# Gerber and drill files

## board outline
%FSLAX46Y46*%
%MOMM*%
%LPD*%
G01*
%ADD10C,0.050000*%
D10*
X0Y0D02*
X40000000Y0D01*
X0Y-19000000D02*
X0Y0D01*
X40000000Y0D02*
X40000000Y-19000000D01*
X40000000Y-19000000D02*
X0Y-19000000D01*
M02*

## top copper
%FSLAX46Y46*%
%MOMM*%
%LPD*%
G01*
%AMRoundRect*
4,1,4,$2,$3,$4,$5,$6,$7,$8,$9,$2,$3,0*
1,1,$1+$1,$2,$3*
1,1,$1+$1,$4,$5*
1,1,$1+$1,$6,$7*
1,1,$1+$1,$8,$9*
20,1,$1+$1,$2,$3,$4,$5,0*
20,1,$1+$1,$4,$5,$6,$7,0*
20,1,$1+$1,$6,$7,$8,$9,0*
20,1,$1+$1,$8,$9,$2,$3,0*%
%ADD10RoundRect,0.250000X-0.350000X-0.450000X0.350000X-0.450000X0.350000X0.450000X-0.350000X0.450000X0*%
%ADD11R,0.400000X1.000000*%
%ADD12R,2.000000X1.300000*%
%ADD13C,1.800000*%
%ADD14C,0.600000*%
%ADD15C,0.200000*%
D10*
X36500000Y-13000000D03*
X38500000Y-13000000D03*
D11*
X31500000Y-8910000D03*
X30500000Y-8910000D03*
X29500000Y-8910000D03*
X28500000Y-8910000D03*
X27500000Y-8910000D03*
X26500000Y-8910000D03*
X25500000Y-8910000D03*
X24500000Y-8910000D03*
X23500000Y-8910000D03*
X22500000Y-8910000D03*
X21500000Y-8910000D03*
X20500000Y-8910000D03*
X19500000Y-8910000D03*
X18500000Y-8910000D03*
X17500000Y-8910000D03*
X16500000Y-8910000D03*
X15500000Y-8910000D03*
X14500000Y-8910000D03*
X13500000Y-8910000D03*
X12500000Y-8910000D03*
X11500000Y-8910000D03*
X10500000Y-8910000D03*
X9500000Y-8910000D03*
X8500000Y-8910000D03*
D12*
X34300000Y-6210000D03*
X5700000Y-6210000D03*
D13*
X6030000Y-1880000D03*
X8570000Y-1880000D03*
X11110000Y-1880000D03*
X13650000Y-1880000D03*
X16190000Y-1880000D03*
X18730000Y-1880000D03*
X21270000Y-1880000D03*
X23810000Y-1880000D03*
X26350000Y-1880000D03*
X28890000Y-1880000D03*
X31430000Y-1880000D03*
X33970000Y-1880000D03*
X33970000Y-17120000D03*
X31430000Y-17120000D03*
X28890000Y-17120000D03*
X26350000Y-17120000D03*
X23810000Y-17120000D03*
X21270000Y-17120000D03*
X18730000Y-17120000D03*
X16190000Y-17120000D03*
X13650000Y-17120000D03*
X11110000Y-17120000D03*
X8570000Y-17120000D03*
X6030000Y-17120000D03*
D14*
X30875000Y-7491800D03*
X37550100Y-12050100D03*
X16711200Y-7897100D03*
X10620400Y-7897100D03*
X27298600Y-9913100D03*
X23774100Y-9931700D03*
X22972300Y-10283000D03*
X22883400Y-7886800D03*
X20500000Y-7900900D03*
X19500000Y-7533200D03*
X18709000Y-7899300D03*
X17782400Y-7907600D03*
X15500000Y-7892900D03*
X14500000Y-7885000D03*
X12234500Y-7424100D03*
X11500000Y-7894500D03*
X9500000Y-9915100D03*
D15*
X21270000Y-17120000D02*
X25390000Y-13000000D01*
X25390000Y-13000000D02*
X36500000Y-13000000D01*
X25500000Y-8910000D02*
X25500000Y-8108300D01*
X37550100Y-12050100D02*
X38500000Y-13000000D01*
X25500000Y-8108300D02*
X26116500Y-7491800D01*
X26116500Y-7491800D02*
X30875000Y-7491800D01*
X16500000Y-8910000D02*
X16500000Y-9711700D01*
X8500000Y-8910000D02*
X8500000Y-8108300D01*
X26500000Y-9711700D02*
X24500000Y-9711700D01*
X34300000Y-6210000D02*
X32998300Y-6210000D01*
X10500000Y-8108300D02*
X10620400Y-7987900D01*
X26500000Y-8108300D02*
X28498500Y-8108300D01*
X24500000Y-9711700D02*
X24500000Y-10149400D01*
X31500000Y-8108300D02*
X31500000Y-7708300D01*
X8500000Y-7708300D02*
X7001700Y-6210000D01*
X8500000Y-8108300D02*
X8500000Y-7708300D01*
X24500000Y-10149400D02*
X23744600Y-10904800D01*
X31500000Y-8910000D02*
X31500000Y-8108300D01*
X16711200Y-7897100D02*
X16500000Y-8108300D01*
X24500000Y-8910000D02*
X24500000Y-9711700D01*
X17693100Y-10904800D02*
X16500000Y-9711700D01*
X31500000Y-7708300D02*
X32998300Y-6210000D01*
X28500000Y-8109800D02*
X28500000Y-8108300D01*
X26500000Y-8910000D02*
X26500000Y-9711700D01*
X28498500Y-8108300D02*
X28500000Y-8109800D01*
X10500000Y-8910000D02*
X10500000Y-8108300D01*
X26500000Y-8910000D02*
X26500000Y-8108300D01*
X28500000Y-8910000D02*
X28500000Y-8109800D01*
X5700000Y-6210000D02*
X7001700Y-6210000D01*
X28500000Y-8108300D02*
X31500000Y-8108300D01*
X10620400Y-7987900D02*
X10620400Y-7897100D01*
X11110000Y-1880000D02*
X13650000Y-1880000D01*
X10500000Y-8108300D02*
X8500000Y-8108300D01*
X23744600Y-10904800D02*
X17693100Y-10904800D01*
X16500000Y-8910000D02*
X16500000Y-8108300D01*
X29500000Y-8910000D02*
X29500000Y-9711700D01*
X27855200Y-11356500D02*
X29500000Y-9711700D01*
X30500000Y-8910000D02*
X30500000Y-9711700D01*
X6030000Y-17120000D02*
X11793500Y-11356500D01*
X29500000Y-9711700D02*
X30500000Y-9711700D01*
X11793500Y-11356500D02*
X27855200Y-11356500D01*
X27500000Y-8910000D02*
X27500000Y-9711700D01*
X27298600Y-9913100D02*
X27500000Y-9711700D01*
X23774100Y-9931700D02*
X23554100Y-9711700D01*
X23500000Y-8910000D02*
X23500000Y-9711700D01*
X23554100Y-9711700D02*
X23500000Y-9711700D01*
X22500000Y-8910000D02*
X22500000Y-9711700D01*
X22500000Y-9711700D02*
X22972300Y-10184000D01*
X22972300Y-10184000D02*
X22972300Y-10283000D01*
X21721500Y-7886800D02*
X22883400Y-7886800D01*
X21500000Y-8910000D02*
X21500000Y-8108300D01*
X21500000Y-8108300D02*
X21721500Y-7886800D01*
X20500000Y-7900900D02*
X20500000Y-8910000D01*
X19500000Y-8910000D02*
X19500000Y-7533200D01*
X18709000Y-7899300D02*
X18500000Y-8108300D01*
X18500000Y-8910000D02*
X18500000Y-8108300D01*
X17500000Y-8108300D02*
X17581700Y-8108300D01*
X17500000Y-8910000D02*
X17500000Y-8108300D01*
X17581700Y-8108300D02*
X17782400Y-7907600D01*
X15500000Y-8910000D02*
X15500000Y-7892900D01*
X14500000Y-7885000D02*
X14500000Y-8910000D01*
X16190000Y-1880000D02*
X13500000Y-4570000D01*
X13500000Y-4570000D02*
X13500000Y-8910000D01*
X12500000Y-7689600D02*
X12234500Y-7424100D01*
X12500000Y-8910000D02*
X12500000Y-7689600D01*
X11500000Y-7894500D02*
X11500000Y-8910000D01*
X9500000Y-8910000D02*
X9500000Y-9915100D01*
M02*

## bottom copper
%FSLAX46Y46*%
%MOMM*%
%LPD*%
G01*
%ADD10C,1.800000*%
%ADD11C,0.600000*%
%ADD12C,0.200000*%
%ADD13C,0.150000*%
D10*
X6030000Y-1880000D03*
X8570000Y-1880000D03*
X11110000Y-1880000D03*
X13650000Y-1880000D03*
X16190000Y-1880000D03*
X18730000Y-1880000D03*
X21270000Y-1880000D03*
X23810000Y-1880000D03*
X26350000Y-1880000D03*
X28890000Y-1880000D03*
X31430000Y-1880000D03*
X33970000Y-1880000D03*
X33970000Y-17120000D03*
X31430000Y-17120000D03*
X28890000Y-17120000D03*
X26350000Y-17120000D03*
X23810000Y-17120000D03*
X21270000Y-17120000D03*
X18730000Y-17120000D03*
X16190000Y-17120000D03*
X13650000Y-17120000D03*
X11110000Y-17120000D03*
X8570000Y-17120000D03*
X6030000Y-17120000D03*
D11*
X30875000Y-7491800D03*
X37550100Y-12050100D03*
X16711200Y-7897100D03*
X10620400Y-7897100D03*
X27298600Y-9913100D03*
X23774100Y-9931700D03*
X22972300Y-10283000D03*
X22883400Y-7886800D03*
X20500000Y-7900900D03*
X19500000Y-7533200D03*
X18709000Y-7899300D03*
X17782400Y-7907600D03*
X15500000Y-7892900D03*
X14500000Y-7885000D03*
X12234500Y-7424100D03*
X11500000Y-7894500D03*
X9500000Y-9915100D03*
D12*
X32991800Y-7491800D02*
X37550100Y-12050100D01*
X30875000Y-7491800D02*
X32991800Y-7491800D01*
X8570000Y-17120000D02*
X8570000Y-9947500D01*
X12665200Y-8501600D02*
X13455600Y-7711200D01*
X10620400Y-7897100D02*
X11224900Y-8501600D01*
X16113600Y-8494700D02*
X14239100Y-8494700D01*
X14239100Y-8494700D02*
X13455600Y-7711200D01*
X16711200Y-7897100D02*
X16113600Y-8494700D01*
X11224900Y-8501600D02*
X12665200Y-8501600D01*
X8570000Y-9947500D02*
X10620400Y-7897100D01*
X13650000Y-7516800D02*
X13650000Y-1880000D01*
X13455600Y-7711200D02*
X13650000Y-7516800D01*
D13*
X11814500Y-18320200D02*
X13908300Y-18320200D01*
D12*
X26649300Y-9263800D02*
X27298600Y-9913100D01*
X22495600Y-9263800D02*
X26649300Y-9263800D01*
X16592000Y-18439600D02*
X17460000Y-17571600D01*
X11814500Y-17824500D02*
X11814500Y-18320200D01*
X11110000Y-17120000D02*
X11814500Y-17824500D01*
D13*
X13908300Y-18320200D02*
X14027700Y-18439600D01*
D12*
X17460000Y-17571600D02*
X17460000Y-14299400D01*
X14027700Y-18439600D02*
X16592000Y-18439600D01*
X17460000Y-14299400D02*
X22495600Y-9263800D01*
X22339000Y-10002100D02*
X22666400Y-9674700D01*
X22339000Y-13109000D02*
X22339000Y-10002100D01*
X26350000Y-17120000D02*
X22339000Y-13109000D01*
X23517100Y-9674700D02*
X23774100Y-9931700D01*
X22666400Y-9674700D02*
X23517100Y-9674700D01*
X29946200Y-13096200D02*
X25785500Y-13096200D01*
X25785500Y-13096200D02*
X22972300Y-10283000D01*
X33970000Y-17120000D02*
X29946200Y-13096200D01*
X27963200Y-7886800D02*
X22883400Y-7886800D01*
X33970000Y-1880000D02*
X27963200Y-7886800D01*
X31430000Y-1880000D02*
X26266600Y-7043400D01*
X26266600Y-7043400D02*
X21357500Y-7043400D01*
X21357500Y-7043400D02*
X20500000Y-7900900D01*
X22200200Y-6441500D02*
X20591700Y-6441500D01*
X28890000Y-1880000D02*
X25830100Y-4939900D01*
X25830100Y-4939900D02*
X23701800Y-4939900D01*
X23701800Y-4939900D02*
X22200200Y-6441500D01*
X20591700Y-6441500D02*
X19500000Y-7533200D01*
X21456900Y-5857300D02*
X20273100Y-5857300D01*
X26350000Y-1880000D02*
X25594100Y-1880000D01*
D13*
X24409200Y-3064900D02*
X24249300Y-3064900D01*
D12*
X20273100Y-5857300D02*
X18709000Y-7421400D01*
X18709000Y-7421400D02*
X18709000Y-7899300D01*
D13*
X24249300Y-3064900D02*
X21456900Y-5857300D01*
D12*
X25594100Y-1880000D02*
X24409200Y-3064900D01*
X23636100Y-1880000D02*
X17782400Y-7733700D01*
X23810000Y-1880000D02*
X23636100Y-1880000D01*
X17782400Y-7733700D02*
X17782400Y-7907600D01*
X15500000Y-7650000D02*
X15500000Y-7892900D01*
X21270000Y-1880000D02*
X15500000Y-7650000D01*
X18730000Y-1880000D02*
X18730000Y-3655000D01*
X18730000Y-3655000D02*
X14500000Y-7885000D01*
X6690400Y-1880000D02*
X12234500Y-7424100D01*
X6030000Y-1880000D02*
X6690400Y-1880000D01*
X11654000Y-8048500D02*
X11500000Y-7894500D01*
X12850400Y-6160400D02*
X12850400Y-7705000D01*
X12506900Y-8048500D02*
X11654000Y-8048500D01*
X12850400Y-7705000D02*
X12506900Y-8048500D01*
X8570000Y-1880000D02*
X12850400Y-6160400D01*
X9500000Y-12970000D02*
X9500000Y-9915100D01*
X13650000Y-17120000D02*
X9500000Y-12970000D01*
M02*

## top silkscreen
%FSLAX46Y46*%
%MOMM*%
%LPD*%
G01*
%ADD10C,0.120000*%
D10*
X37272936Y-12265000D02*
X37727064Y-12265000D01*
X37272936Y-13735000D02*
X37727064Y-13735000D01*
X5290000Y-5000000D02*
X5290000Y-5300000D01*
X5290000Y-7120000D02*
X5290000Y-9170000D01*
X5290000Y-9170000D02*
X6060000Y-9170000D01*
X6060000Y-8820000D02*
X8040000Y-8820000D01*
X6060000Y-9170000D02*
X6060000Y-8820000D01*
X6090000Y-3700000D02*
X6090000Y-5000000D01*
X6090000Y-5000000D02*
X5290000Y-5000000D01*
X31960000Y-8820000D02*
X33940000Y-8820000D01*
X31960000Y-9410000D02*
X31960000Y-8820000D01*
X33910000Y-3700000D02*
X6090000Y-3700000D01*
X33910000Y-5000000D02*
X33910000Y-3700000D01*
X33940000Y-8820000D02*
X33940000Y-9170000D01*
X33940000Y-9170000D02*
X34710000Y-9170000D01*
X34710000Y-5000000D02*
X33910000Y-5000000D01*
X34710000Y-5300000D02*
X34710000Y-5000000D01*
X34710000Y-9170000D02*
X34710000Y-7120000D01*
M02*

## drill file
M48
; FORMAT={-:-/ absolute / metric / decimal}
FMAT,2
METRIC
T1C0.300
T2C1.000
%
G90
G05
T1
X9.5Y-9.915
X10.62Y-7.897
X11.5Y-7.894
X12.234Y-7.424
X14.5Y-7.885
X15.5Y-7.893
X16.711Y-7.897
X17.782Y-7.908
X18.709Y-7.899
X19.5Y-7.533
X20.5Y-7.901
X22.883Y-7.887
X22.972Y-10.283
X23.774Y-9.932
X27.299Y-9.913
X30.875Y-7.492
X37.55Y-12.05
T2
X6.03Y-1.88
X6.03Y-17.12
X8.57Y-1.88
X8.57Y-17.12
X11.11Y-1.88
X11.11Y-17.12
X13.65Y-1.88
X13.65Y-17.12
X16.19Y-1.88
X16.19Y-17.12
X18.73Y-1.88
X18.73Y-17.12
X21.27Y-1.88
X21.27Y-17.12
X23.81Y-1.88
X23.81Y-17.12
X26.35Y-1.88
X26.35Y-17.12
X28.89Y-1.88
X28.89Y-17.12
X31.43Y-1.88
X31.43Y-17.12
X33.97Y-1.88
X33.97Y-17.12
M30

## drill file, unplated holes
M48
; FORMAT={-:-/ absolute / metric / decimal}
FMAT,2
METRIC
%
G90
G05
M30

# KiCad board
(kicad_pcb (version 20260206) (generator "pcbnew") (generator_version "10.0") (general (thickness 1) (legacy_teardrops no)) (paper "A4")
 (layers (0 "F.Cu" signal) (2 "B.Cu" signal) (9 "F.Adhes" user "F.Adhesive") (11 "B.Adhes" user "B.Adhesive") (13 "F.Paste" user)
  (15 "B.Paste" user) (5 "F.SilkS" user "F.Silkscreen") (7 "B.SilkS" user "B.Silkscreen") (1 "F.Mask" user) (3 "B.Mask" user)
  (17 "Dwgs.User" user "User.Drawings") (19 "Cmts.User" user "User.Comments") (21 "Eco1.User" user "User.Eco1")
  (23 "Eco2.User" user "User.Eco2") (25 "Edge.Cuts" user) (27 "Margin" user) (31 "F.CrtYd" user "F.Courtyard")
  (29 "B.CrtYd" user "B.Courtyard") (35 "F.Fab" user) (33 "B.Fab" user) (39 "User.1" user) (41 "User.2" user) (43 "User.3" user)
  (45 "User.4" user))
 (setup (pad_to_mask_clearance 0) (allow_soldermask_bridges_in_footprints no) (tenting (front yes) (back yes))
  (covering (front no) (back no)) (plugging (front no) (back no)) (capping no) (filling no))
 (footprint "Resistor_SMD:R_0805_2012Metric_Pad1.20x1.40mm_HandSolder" (layer "F.Cu") (at 37.5 13)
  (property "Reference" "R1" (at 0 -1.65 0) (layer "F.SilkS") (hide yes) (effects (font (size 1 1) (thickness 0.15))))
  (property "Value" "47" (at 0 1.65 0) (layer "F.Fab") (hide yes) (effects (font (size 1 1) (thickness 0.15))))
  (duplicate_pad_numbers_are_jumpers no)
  (fp_line (start -0.227064 -0.735) (end 0.227064 -0.735) (stroke (width 0.12) (type solid)) (layer "F.SilkS"))
  (fp_line (start -0.227064 0.735) (end 0.227064 0.735) (stroke (width 0.12) (type solid)) (layer "F.SilkS"))
  (pad "1" smd roundrect (at -1 0) (size 1.2 1.4) (layers "F.Cu" "F.Mask" "F.Paste") (roundrect_rratio 0.208333) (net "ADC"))
  (pad "2" smd roundrect (at 1 0) (size 1.2 1.4) (layers "F.Cu" "F.Mask" "F.Paste") (roundrect_rratio 0.208333) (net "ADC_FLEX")))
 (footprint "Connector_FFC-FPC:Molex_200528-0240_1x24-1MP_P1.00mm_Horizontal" (layer "F.Cu") (at 20 8 180)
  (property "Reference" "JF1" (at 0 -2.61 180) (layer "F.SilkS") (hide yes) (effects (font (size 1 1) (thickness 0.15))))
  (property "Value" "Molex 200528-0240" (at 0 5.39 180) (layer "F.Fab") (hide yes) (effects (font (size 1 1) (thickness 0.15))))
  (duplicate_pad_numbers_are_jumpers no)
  (fp_line (start 14.71 3) (end 14.71 2.7) (stroke (width 0.12) (type solid)) (layer "F.SilkS"))
  (fp_line (start 14.71 0.88) (end 14.71 -1.17) (stroke (width 0.12) (type solid)) (layer "F.SilkS"))
  (fp_line (start 14.71 -1.17) (end 13.94 -1.17) (stroke (width 0.12) (type solid)) (layer "F.SilkS"))
  (fp_line (start 13.94 -0.82) (end 11.96 -0.82) (stroke (width 0.12) (type solid)) (layer "F.SilkS"))
  (fp_line (start 13.94 -1.17) (end 13.94 -0.82) (stroke (width 0.12) (type solid)) (layer "F.SilkS"))
  (fp_line (start 13.91 4.3) (end 13.91 3) (stroke (width 0.12) (type solid)) (layer "F.SilkS"))
  (fp_line (start 13.91 3) (end 14.71 3) (stroke (width 0.12) (type solid)) (layer "F.SilkS"))
  (fp_line (start -11.96 -0.82) (end -13.94 -0.82) (stroke (width 0.12) (type solid)) (layer "F.SilkS"))
  (fp_line (start -11.96 -1.41) (end -11.96 -0.82) (stroke (width 0.12) (type solid)) (layer "F.SilkS"))
  (fp_line (start -13.91 4.3) (end 13.91 4.3) (stroke (width 0.12) (type solid)) (layer "F.SilkS"))
  (fp_line (start -13.91 3) (end -13.91 4.3) (stroke (width 0.12) (type solid)) (layer "F.SilkS"))
  (fp_line (start -13.94 -0.82) (end -13.94 -1.17) (stroke (width 0.12) (type solid)) (layer "F.SilkS"))
  (fp_line (start -13.94 -1.17) (end -14.71 -1.17) (stroke (width 0.12) (type solid)) (layer "F.SilkS"))
  (fp_line (start -14.71 3) (end -13.91 3) (stroke (width 0.12) (type solid)) (layer "F.SilkS"))
  (fp_line (start -14.71 2.7) (end -14.71 3) (stroke (width 0.12) (type solid)) (layer "F.SilkS"))
  (fp_line (start -14.71 -1.17) (end -14.71 0.88) (stroke (width 0.12) (type solid)) (layer "F.SilkS"))
  (pad "1" smd rect (at -11.5 -0.91 180) (size 0.4 1) (layers "F.Cu" "F.Mask" "F.Paste") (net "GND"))
  (pad "2" smd rect (at -10.5 -0.91 180) (size 0.4 1) (layers "F.Cu" "F.Mask" "F.Paste") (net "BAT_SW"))
  (pad "3" smd rect (at -9.5 -0.91 180) (size 0.4 1) (layers "F.Cu" "F.Mask" "F.Paste") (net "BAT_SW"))
  (pad "4" smd rect (at -8.5 -0.91 180) (size 0.4 1) (layers "F.Cu" "F.Mask" "F.Paste") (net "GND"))
  (pad "5" smd rect (at -7.5 -0.91 180) (size 0.4 1) (layers "F.Cu" "F.Mask" "F.Paste") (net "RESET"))
  (pad "6" smd rect (at -6.5 -0.91 180) (size 0.4 1) (layers "F.Cu" "F.Mask" "F.Paste") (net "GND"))
  (pad "7" smd rect (at -5.5 -0.91 180) (size 0.4 1) (layers "F.Cu" "F.Mask" "F.Paste") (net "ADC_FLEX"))
  (pad "8" smd rect (at -4.5 -0.91 180) (size 0.4 1) (layers "F.Cu" "F.Mask" "F.Paste") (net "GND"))
  (pad "9" smd rect (at -3.5 -0.91 180) (size 0.4 1) (layers "F.Cu" "F.Mask" "F.Paste") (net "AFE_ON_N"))
  (pad "10" smd rect (at -2.5 -0.91 180) (size 0.4 1) (layers "F.Cu" "F.Mask" "F.Paste") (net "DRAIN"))
  (pad "11" smd rect (at -1.5 -0.91 180) (size 0.4 1) (layers "F.Cu" "F.Mask" "F.Paste") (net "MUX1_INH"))
  (pad "12" smd rect (at -0.5 -0.91 180) (size 0.4 1) (layers "F.Cu" "F.Mask" "F.Paste") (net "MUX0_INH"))
  (pad "13" smd rect (at 0.5 -0.91 180) (size 0.4 1) (layers "F.Cu" "F.Mask" "F.Paste") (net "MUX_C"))
  (pad "14" smd rect (at 1.5 -0.91 180) (size 0.4 1) (layers "F.Cu" "F.Mask" "F.Paste") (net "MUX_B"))
  (pad "15" smd rect (at 2.5 -0.91 180) (size 0.4 1) (layers "F.Cu" "F.Mask" "F.Paste") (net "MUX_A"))
  (pad "16" smd rect (at 3.5 -0.91 180) (size 0.4 1) (layers "F.Cu" "F.Mask" "F.Paste") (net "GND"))
  (pad "17" smd rect (at 4.5 -0.91 180) (size 0.4 1) (layers "F.Cu" "F.Mask" "F.Paste") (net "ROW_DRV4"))
  (pad "18" smd rect (at 5.5 -0.91 180) (size 0.4 1) (layers "F.Cu" "F.Mask" "F.Paste") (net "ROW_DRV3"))
  (pad "19" smd rect (at 6.5 -0.91 180) (size 0.4 1) (layers "F.Cu" "F.Mask" "F.Paste") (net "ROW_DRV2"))
  (pad "20" smd rect (at 7.5 -0.91 180) (size 0.4 1) (layers "F.Cu" "F.Mask" "F.Paste") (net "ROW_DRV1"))
  (pad "21" smd rect (at 8.5 -0.91 180) (size 0.4 1) (layers "F.Cu" "F.Mask" "F.Paste") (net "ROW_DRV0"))
  (pad "22" smd rect (at 9.5 -0.91 180) (size 0.4 1) (layers "F.Cu" "F.Mask" "F.Paste") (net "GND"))
  (pad "23" smd rect (at 10.5 -0.91 180) (size 0.4 1) (layers "F.Cu" "F.Mask" "F.Paste") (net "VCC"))
  (pad "24" smd rect (at 11.5 -0.91 180) (size 0.4 1) (layers "F.Cu" "F.Mask" "F.Paste") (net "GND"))
  (pad "MP" smd rect (at -14.3 1.79 180) (size 2 1.3) (layers "F.Cu" "F.Mask" "F.Paste") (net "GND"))
  (pad "MP" smd rect (at 14.3 1.79 180) (size 2 1.3) (layers "F.Cu" "F.Mask" "F.Paste") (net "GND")))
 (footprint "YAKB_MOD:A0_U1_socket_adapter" (layer "F.Cu") (at 0 0)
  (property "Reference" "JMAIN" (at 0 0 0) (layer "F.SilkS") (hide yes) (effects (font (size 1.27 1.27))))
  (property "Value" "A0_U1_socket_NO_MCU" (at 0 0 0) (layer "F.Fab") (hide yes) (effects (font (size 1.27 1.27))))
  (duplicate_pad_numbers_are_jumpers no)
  (pad "1" thru_hole circle (at 6.03 1.88) (size 1.8 1.8) (drill 1) (layers "*.Cu" "*.Mask") (remove_unused_layers no) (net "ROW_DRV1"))
  (pad "2" thru_hole circle (at 8.57 1.88) (size 1.8 1.8) (drill 1) (layers "*.Cu" "*.Mask") (remove_unused_layers no) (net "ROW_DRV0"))
  (pad "3" thru_hole circle (at 11.11 1.88) (size 1.8 1.8) (drill 1) (layers "*.Cu" "*.Mask") (remove_unused_layers no) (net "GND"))
  (pad "4" thru_hole circle (at 13.65 1.88) (size 1.8 1.8) (drill 1) (layers "*.Cu" "*.Mask") (remove_unused_layers no) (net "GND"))
  (pad "5" thru_hole circle (at 16.19 1.88) (size 1.8 1.8) (drill 1) (layers "*.Cu" "*.Mask") (remove_unused_layers no) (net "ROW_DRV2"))
  (pad "6" thru_hole circle (at 18.73 1.88) (size 1.8 1.8) (drill 1) (layers "*.Cu" "*.Mask") (remove_unused_layers no) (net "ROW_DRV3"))
  (pad "7" thru_hole circle (at 21.27 1.88) (size 1.8 1.8) (drill 1) (layers "*.Cu" "*.Mask") (remove_unused_layers no) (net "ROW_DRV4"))
  (pad "8" thru_hole circle (at 23.81 1.88) (size 1.8 1.8) (drill 1) (layers "*.Cu" "*.Mask") (remove_unused_layers no) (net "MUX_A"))
  (pad "9" thru_hole circle (at 26.35 1.88) (size 1.8 1.8) (drill 1) (layers "*.Cu" "*.Mask") (remove_unused_layers no) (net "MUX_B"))
  (pad "10" thru_hole circle (at 28.89 1.88) (size 1.8 1.8) (drill 1) (layers "*.Cu" "*.Mask") (remove_unused_layers no) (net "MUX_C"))
  (pad "11" thru_hole circle (at 31.43 1.88) (size 1.8 1.8) (drill 1) (layers "*.Cu" "*.Mask") (remove_unused_layers no) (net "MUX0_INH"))
  (pad "12" thru_hole circle (at 33.97 1.88) (size 1.8 1.8) (drill 1) (layers "*.Cu" "*.Mask") (remove_unused_layers no) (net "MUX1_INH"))
  (pad "13" thru_hole circle (at 33.97 17.12) (size 1.8 1.8) (drill 1) (layers "*.Cu" "*.Mask") (remove_unused_layers no) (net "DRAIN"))
  (pad "14" thru_hole circle (at 31.43 17.12) (size 1.8 1.8) (drill 1) (layers "*.Cu" "*.Mask") (remove_unused_layers no)
   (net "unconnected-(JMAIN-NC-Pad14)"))
  (pad "15" thru_hole circle (at 28.89 17.12) (size 1.8 1.8) (drill 1) (layers "*.Cu" "*.Mask") (remove_unused_layers no)
   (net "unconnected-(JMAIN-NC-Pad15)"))
  (pad "16" thru_hole circle (at 26.35 17.12) (size 1.8 1.8) (drill 1) (layers "*.Cu" "*.Mask") (remove_unused_layers no) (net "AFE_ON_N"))
  (pad "17" thru_hole circle (at 23.81 17.12) (size 1.8 1.8) (drill 1) (layers "*.Cu" "*.Mask") (remove_unused_layers no)
   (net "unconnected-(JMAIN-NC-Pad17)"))
  (pad "18" thru_hole circle (at 21.27 17.12) (size 1.8 1.8) (drill 1) (layers "*.Cu" "*.Mask") (remove_unused_layers no) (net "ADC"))
  (pad "19" thru_hole circle (at 18.73 17.12) (size 1.8 1.8) (drill 1) (layers "*.Cu" "*.Mask") (remove_unused_layers no)
   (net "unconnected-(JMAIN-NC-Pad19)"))
  (pad "20" thru_hole circle (at 16.19 17.12) (size 1.8 1.8) (drill 1) (layers "*.Cu" "*.Mask") (remove_unused_layers no)
   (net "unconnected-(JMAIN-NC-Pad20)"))
  (pad "21" thru_hole circle (at 13.65 17.12) (size 1.8 1.8) (drill 1) (layers "*.Cu" "*.Mask") (remove_unused_layers no) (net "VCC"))
  (pad "22" thru_hole circle (at 11.11 17.12) (size 1.8 1.8) (drill 1) (layers "*.Cu" "*.Mask") (remove_unused_layers no) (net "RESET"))
  (pad "23" thru_hole circle (at 8.57 17.12) (size 1.8 1.8) (drill 1) (layers "*.Cu" "*.Mask") (remove_unused_layers no) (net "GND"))
  (pad "24" thru_hole circle (at 6.03 17.12) (size 1.8 1.8) (drill 1) (layers "*.Cu" "*.Mask") (remove_unused_layers no) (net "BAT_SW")))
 (gr_line (start 0 0) (end 40 0) (stroke (width 0.05) (type default)) (layer "Edge.Cuts"))
 (gr_line (start 0 19) (end 0 0) (stroke (width 0.05) (type default)) (layer "Edge.Cuts"))
 (gr_line (start 40 0) (end 40 19) (stroke (width 0.05) (type default)) (layer "Edge.Cuts"))
 (gr_line (start 40 19) (end 0 19) (stroke (width 0.05) (type default)) (layer "Edge.Cuts"))
 (segment (start 21.27 17.12) (end 25.39 13) (width 0.2) (layer "F.Cu") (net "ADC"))
 (segment (start 25.39 13) (end 36.5 13) (width 0.2) (layer "F.Cu") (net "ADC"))
 (segment (start 25.5 8.91) (end 25.5 8.1083) (width 0.2) (layer "F.Cu") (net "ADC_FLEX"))
 (segment (start 37.5501 12.0501) (end 38.5 13) (width 0.2) (layer "F.Cu") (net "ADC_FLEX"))
 (segment (start 25.5 8.1083) (end 26.1165 7.4918) (width 0.2) (layer "F.Cu") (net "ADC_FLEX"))
 (segment (start 26.1165 7.4918) (end 30.875 7.4918) (width 0.2) (layer "F.Cu") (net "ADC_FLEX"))
 (via (at 30.875 7.4918) (size 0.6) (drill 0.3) (layers "F.Cu" "B.Cu") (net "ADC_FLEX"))
 (via (at 37.5501 12.0501) (size 0.6) (drill 0.3) (layers "F.Cu" "B.Cu") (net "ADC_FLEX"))
 (segment (start 32.9918 7.4918) (end 37.5501 12.0501) (width 0.2) (layer "B.Cu") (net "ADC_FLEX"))
 (segment (start 30.875 7.4918) (end 32.9918 7.4918) (width 0.2) (layer "B.Cu") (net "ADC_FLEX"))
 (segment (start 16.5 8.91) (end 16.5 9.7117) (width 0.2) (layer "F.Cu") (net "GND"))
 (segment (start 8.5 8.91) (end 8.5 8.1083) (width 0.2) (layer "F.Cu") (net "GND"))
 (segment (start 26.5 9.7117) (end 24.5 9.7117) (width 0.2) (layer "F.Cu") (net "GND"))
 (segment (start 34.3 6.21) (end 32.9983 6.21) (width 0.2) (layer "F.Cu") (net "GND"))
 (segment (start 10.5 8.1083) (end 10.6204 7.9879) (width 0.2) (layer "F.Cu") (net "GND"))
 (segment (start 26.5 8.1083) (end 28.4985 8.1083) (width 0.2) (layer "F.Cu") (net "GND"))
 (segment (start 24.5 9.7117) (end 24.5 10.1494) (width 0.2) (layer "F.Cu") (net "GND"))
 (segment (start 31.5 8.1083) (end 31.5 7.7083) (width 0.2) (layer "F.Cu") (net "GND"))
 (segment (start 8.5 7.7083) (end 7.0017 6.21) (width 0.2) (layer "F.Cu") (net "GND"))
 (segment (start 8.5 8.1083) (end 8.5 7.7083) (width 0.2) (layer "F.Cu") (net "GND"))
 (segment (start 24.5 10.1494) (end 23.7446 10.9048) (width 0.2) (layer "F.Cu") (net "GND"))
 (segment (start 31.5 8.91) (end 31.5 8.1083) (width 0.2) (layer "F.Cu") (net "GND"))
 (segment (start 16.7112 7.8971) (end 16.5 8.1083) (width 0.2) (layer "F.Cu") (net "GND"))
 (segment (start 24.5 8.91) (end 24.5 9.7117) (width 0.2) (layer "F.Cu") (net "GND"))
 (segment (start 17.6931 10.9048) (end 16.5 9.7117) (width 0.2) (layer "F.Cu") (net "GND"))
 (segment (start 31.5 7.7083) (end 32.9983 6.21) (width 0.2) (layer "F.Cu") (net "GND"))
 (segment (start 28.5 8.1098) (end 28.5 8.1083) (width 0.2) (layer "F.Cu") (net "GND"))
 (segment (start 26.5 8.91) (end 26.5 9.7117) (width 0.2) (layer "F.Cu") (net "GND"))
 (segment (start 28.4985 8.1083) (end 28.5 8.1098) (width 0.2) (layer "F.Cu") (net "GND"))
 (segment (start 10.5 8.91) (end 10.5 8.1083) (width 0.2) (layer "F.Cu") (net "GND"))
 (segment (start 26.5 8.91) (end 26.5 8.1083) (width 0.2) (layer "F.Cu") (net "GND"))
 (segment (start 28.5 8.91) (end 28.5 8.1098) (width 0.2) (layer "F.Cu") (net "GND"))
 (segment (start 5.7 6.21) (end 7.0017 6.21) (width 0.2) (layer "F.Cu") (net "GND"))
 (segment (start 28.5 8.1083) (end 31.5 8.1083) (width 0.2) (layer "F.Cu") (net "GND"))
 (segment (start 10.6204 7.9879) (end 10.6204 7.8971) (width 0.2) (layer "F.Cu") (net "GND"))
 (segment (start 11.11 1.88) (end 13.65 1.88) (width 0.2) (layer "F.Cu") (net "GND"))
 (segment (start 10.5 8.1083) (end 8.5 8.1083) (width 0.2) (layer "F.Cu") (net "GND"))
 (segment (start 23.7446 10.9048) (end 17.6931 10.9048) (width 0.2) (layer "F.Cu") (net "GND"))
 (segment (start 16.5 8.91) (end 16.5 8.1083) (width 0.2) (layer "F.Cu") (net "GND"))
 (via (at 16.7112 7.8971) (size 0.6) (drill 0.3) (layers "F.Cu" "B.Cu") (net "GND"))
 (via (at 10.6204 7.8971) (size 0.6) (drill 0.3) (layers "F.Cu" "B.Cu") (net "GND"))
 (segment (start 8.57 17.12) (end 8.57 9.9475) (width 0.2) (layer "B.Cu") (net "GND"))
 (segment (start 12.6652 8.5016) (end 13.4556 7.7112) (width 0.2) (layer "B.Cu") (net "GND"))
 (segment (start 10.6204 7.8971) (end 11.2249 8.5016) (width 0.2) (layer "B.Cu") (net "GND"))
 (segment (start 16.1136 8.4947) (end 14.2391 8.4947) (width 0.2) (layer "B.Cu") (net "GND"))
 (segment (start 14.2391 8.4947) (end 13.4556 7.7112) (width 0.2) (layer "B.Cu") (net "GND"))
 (segment (start 16.7112 7.8971) (end 16.1136 8.4947) (width 0.2) (layer "B.Cu") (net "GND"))
 (segment (start 11.2249 8.5016) (end 12.6652 8.5016) (width 0.2) (layer "B.Cu") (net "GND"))
 (segment (start 8.57 9.9475) (end 10.6204 7.8971) (width 0.2) (layer "B.Cu") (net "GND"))
 (segment (start 13.65 7.5168) (end 13.65 1.88) (width 0.2) (layer "B.Cu") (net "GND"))
 (segment (start 13.4556 7.7112) (end 13.65 7.5168) (width 0.2) (layer "B.Cu") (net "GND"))
 (segment (start 29.5 8.91) (end 29.5 9.7117) (width 0.2) (layer "F.Cu") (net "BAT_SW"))
 (segment (start 27.8552 11.3565) (end 29.5 9.7117) (width 0.2) (layer "F.Cu") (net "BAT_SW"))
 (segment (start 30.5 8.91) (end 30.5 9.7117) (width 0.2) (layer "F.Cu") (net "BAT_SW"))
 (segment (start 6.03 17.12) (end 11.7935 11.3565) (width 0.2) (layer "F.Cu") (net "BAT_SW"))
 (segment (start 29.5 9.7117) (end 30.5 9.7117) (width 0.2) (layer "F.Cu") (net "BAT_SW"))
 (segment (start 11.7935 11.3565) (end 27.8552 11.3565) (width 0.2) (layer "F.Cu") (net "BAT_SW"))
 (segment (start 27.5 8.91) (end 27.5 9.7117) (width 0.2) (layer "F.Cu") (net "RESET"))
 (segment (start 27.2986 9.9131) (end 27.5 9.7117) (width 0.2) (layer "F.Cu") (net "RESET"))
 (via (at 27.2986 9.9131) (size 0.6) (drill 0.3) (layers "F.Cu" "B.Cu") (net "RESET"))
 (segment (start 11.8145 18.3202) (end 13.9083 18.3202) (width 0.15) (layer "B.Cu") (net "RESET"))
 (segment (start 26.6493 9.2638) (end 27.2986 9.9131) (width 0.2) (layer "B.Cu") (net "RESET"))
 (segment (start 22.4956 9.2638) (end 26.6493 9.2638) (width 0.2) (layer "B.Cu") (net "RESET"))
 (segment (start 16.592 18.4396) (end 17.46 17.5716) (width 0.2) (layer "B.Cu") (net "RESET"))
 (segment (start 11.8145 17.8245) (end 11.8145 18.3202) (width 0.2) (layer "B.Cu") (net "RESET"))
 (segment (start 11.11 17.12) (end 11.8145 17.8245) (width 0.2) (layer "B.Cu") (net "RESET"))
 (segment (start 13.9083 18.3202) (end 14.0277 18.4396) (width 0.15) (layer "B.Cu") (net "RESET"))
 (segment (start 17.46 17.5716) (end 17.46 14.2994) (width 0.2) (layer "B.Cu") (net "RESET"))
 (segment (start 14.0277 18.4396) (end 16.592 18.4396) (width 0.2) (layer "B.Cu") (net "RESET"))
 (segment (start 17.46 14.2994) (end 22.4956 9.2638) (width 0.2) (layer "B.Cu") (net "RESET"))
 (segment (start 23.7741 9.9317) (end 23.5541 9.7117) (width 0.2) (layer "F.Cu") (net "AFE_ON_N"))
 (segment (start 23.5 8.91) (end 23.5 9.7117) (width 0.2) (layer "F.Cu") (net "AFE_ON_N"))
 (segment (start 23.5541 9.7117) (end 23.5 9.7117) (width 0.2) (layer "F.Cu") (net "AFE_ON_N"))
 (via (at 23.7741 9.9317) (size 0.6) (drill 0.3) (layers "F.Cu" "B.Cu") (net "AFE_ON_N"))
 (segment (start 22.339 10.0021) (end 22.6664 9.6747) (width 0.2) (layer "B.Cu") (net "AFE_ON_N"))
 (segment (start 22.339 13.109) (end 22.339 10.0021) (width 0.2) (layer "B.Cu") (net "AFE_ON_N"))
 (segment (start 26.35 17.12) (end 22.339 13.109) (width 0.2) (layer "B.Cu") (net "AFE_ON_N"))
 (segment (start 23.5171 9.6747) (end 23.7741 9.9317) (width 0.2) (layer "B.Cu") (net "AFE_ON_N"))
 (segment (start 22.6664 9.6747) (end 23.5171 9.6747) (width 0.2) (layer "B.Cu") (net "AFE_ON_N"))
 (segment (start 22.5 8.91) (end 22.5 9.7117) (width 0.2) (layer "F.Cu") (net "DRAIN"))
 (segment (start 22.5 9.7117) (end 22.9723 10.184) (width 0.2) (layer "F.Cu") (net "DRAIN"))
 (segment (start 22.9723 10.184) (end 22.9723 10.283) (width 0.2) (layer "F.Cu") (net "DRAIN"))
 (via (at 22.9723 10.283) (size 0.6) (drill 0.3) (layers "F.Cu" "B.Cu") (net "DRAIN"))
 (segment (start 29.9462 13.0962) (end 25.7855 13.0962) (width 0.2) (layer "B.Cu") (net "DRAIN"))
 (segment (start 25.7855 13.0962) (end 22.9723 10.283) (width 0.2) (layer "B.Cu") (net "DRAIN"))
 (segment (start 33.97 17.12) (end 29.9462 13.0962) (width 0.2) (layer "B.Cu") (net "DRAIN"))
 (segment (start 21.7215 7.8868) (end 22.8834 7.8868) (width 0.2) (layer "F.Cu") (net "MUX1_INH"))
 (segment (start 21.5 8.91) (end 21.5 8.1083) (width 0.2) (layer "F.Cu") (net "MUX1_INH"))
 (segment (start 21.5 8.1083) (end 21.7215 7.8868) (width 0.2) (layer "F.Cu") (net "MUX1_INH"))
 (via (at 22.8834 7.8868) (size 0.6) (drill 0.3) (layers "F.Cu" "B.Cu") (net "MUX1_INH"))
 (segment (start 27.9632 7.8868) (end 22.8834 7.8868) (width 0.2) (layer "B.Cu") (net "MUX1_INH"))
 (segment (start 33.97 1.88) (end 27.9632 7.8868) (width 0.2) (layer "B.Cu") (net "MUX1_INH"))
 (segment (start 20.5 7.9009) (end 20.5 8.91) (width 0.2) (layer "F.Cu") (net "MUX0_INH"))
 (via (at 20.5 7.9009) (size 0.6) (drill 0.3) (layers "F.Cu" "B.Cu") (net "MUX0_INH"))
 (segment (start 31.43 1.88) (end 26.2666 7.0434) (width 0.2) (layer "B.Cu") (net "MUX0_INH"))
 (segment (start 26.2666 7.0434) (end 21.3575 7.0434) (width 0.2) (layer "B.Cu") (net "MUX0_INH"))
 (segment (start 21.3575 7.0434) (end 20.5 7.9009) (width 0.2) (layer "B.Cu") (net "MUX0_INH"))
 (segment (start 19.5 8.91) (end 19.5 7.5332) (width 0.2) (layer "F.Cu") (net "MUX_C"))
 (via (at 19.5 7.5332) (size 0.6) (drill 0.3) (layers "F.Cu" "B.Cu") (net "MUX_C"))
 (segment (start 22.2002 6.4415) (end 20.5917 6.4415) (width 0.2) (layer "B.Cu") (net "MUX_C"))
 (segment (start 28.89 1.88) (end 25.8301 4.9399) (width 0.2) (layer "B.Cu") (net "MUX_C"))
 (segment (start 25.8301 4.9399) (end 23.7018 4.9399) (width 0.2) (layer "B.Cu") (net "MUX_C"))
 (segment (start 23.7018 4.9399) (end 22.2002 6.4415) (width 0.2) (layer "B.Cu") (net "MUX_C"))
 (segment (start 20.5917 6.4415) (end 19.5 7.5332) (width 0.2) (layer "B.Cu") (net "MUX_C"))
 (segment (start 18.709 7.8993) (end 18.5 8.1083) (width 0.2) (layer "F.Cu") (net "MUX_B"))
 (segment (start 18.5 8.91) (end 18.5 8.1083) (width 0.2) (layer "F.Cu") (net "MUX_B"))
 (via (at 18.709 7.8993) (size 0.6) (drill 0.3) (layers "F.Cu" "B.Cu") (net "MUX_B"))
 (segment (start 21.4569 5.8573) (end 20.2731 5.8573) (width 0.2) (layer "B.Cu") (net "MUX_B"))
 (segment (start 26.35 1.88) (end 25.5941 1.88) (width 0.2) (layer "B.Cu") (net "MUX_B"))
 (segment (start 24.4092 3.0649) (end 24.2493 3.0649) (width 0.15) (layer "B.Cu") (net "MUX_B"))
 (segment (start 20.2731 5.8573) (end 18.709 7.4214) (width 0.2) (layer "B.Cu") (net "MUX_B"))
 (segment (start 18.709 7.4214) (end 18.709 7.8993) (width 0.2) (layer "B.Cu") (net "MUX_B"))
 (segment (start 24.2493 3.0649) (end 21.4569 5.8573) (width 0.15) (layer "B.Cu") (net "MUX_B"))
 (segment (start 25.5941 1.88) (end 24.4092 3.0649) (width 0.2) (layer "B.Cu") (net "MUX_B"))
 (segment (start 17.5 8.1083) (end 17.5817 8.1083) (width 0.2) (layer "F.Cu") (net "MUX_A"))
 (segment (start 17.5 8.91) (end 17.5 8.1083) (width 0.2) (layer "F.Cu") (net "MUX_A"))
 (segment (start 17.5817 8.1083) (end 17.7824 7.9076) (width 0.2) (layer "F.Cu") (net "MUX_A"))
 (via (at 17.7824 7.9076) (size 0.6) (drill 0.3) (layers "F.Cu" "B.Cu") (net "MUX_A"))
 (segment (start 23.6361 1.88) (end 17.7824 7.7337) (width 0.2) (layer "B.Cu") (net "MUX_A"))
 (segment (start 23.81 1.88) (end 23.6361 1.88) (width 0.2) (layer "B.Cu") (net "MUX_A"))
 (segment (start 17.7824 7.7337) (end 17.7824 7.9076) (width 0.2) (layer "B.Cu") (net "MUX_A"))
 (segment (start 15.5 8.91) (end 15.5 7.8929) (width 0.2) (layer "F.Cu") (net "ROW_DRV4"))
 (via (at 15.5 7.8929) (size 0.6) (drill 0.3) (layers "F.Cu" "B.Cu") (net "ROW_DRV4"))
 (segment (start 15.5 7.65) (end 15.5 7.8929) (width 0.2) (layer "B.Cu") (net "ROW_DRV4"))
 (segment (start 21.27 1.88) (end 15.5 7.65) (width 0.2) (layer "B.Cu") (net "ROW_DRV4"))
 (segment (start 14.5 7.885) (end 14.5 8.91) (width 0.2) (layer "F.Cu") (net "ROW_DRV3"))
 (via (at 14.5 7.885) (size 0.6) (drill 0.3) (layers "F.Cu" "B.Cu") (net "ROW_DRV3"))
 (segment (start 18.73 1.88) (end 18.73 3.655) (width 0.2) (layer "B.Cu") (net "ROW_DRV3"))
 (segment (start 18.73 3.655) (end 14.5 7.885) (width 0.2) (layer "B.Cu") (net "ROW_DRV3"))
 (segment (start 16.19 1.88) (end 13.5 4.57) (width 0.2) (layer "F.Cu") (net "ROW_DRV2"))
 (segment (start 13.5 4.57) (end 13.5 8.91) (width 0.2) (layer "F.Cu") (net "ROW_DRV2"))
 (segment (start 12.5 7.6896) (end 12.2345 7.4241) (width 0.2) (layer "F.Cu") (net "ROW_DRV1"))
 (segment (start 12.5 8.91) (end 12.5 7.6896) (width 0.2) (layer "F.Cu") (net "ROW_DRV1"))
 (via (at 12.2345 7.4241) (size 0.6) (drill 0.3) (layers "F.Cu" "B.Cu") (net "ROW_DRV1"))
 (segment (start 6.6904 1.88) (end 12.2345 7.4241) (width 0.2) (layer "B.Cu") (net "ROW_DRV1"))
 (segment (start 6.03 1.88) (end 6.6904 1.88) (width 0.2) (layer "B.Cu") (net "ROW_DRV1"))
 (segment (start 11.5 7.8945) (end 11.5 8.91) (width 0.2) (layer "F.Cu") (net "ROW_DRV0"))
 (via (at 11.5 7.8945) (size 0.6) (drill 0.3) (layers "F.Cu" "B.Cu") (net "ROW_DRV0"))
 (segment (start 11.654 8.0485) (end 11.5 7.8945) (width 0.2) (layer "B.Cu") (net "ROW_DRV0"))
 (segment (start 12.8504 6.1604) (end 12.8504 7.705) (width 0.2) (layer "B.Cu") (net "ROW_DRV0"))
 (segment (start 12.5069 8.0485) (end 11.654 8.0485) (width 0.2) (layer "B.Cu") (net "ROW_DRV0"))
 (segment (start 12.8504 7.705) (end 12.5069 8.0485) (width 0.2) (layer "B.Cu") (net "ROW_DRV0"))
 (segment (start 8.57 1.88) (end 12.8504 6.1604) (width 0.2) (layer "B.Cu") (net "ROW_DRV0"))
 (segment (start 9.5 8.91) (end 9.5 9.9151) (width 0.2) (layer "F.Cu") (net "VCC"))
 (via (at 9.5 9.9151) (size 0.6) (drill 0.3) (layers "F.Cu" "B.Cu") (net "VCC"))
 (segment (start 9.5 12.97) (end 9.5 9.9151) (width 0.2) (layer "B.Cu") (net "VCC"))
 (segment (start 13.65 17.12) (end 9.5 12.97) (width 0.2) (layer "B.Cu") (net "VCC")))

